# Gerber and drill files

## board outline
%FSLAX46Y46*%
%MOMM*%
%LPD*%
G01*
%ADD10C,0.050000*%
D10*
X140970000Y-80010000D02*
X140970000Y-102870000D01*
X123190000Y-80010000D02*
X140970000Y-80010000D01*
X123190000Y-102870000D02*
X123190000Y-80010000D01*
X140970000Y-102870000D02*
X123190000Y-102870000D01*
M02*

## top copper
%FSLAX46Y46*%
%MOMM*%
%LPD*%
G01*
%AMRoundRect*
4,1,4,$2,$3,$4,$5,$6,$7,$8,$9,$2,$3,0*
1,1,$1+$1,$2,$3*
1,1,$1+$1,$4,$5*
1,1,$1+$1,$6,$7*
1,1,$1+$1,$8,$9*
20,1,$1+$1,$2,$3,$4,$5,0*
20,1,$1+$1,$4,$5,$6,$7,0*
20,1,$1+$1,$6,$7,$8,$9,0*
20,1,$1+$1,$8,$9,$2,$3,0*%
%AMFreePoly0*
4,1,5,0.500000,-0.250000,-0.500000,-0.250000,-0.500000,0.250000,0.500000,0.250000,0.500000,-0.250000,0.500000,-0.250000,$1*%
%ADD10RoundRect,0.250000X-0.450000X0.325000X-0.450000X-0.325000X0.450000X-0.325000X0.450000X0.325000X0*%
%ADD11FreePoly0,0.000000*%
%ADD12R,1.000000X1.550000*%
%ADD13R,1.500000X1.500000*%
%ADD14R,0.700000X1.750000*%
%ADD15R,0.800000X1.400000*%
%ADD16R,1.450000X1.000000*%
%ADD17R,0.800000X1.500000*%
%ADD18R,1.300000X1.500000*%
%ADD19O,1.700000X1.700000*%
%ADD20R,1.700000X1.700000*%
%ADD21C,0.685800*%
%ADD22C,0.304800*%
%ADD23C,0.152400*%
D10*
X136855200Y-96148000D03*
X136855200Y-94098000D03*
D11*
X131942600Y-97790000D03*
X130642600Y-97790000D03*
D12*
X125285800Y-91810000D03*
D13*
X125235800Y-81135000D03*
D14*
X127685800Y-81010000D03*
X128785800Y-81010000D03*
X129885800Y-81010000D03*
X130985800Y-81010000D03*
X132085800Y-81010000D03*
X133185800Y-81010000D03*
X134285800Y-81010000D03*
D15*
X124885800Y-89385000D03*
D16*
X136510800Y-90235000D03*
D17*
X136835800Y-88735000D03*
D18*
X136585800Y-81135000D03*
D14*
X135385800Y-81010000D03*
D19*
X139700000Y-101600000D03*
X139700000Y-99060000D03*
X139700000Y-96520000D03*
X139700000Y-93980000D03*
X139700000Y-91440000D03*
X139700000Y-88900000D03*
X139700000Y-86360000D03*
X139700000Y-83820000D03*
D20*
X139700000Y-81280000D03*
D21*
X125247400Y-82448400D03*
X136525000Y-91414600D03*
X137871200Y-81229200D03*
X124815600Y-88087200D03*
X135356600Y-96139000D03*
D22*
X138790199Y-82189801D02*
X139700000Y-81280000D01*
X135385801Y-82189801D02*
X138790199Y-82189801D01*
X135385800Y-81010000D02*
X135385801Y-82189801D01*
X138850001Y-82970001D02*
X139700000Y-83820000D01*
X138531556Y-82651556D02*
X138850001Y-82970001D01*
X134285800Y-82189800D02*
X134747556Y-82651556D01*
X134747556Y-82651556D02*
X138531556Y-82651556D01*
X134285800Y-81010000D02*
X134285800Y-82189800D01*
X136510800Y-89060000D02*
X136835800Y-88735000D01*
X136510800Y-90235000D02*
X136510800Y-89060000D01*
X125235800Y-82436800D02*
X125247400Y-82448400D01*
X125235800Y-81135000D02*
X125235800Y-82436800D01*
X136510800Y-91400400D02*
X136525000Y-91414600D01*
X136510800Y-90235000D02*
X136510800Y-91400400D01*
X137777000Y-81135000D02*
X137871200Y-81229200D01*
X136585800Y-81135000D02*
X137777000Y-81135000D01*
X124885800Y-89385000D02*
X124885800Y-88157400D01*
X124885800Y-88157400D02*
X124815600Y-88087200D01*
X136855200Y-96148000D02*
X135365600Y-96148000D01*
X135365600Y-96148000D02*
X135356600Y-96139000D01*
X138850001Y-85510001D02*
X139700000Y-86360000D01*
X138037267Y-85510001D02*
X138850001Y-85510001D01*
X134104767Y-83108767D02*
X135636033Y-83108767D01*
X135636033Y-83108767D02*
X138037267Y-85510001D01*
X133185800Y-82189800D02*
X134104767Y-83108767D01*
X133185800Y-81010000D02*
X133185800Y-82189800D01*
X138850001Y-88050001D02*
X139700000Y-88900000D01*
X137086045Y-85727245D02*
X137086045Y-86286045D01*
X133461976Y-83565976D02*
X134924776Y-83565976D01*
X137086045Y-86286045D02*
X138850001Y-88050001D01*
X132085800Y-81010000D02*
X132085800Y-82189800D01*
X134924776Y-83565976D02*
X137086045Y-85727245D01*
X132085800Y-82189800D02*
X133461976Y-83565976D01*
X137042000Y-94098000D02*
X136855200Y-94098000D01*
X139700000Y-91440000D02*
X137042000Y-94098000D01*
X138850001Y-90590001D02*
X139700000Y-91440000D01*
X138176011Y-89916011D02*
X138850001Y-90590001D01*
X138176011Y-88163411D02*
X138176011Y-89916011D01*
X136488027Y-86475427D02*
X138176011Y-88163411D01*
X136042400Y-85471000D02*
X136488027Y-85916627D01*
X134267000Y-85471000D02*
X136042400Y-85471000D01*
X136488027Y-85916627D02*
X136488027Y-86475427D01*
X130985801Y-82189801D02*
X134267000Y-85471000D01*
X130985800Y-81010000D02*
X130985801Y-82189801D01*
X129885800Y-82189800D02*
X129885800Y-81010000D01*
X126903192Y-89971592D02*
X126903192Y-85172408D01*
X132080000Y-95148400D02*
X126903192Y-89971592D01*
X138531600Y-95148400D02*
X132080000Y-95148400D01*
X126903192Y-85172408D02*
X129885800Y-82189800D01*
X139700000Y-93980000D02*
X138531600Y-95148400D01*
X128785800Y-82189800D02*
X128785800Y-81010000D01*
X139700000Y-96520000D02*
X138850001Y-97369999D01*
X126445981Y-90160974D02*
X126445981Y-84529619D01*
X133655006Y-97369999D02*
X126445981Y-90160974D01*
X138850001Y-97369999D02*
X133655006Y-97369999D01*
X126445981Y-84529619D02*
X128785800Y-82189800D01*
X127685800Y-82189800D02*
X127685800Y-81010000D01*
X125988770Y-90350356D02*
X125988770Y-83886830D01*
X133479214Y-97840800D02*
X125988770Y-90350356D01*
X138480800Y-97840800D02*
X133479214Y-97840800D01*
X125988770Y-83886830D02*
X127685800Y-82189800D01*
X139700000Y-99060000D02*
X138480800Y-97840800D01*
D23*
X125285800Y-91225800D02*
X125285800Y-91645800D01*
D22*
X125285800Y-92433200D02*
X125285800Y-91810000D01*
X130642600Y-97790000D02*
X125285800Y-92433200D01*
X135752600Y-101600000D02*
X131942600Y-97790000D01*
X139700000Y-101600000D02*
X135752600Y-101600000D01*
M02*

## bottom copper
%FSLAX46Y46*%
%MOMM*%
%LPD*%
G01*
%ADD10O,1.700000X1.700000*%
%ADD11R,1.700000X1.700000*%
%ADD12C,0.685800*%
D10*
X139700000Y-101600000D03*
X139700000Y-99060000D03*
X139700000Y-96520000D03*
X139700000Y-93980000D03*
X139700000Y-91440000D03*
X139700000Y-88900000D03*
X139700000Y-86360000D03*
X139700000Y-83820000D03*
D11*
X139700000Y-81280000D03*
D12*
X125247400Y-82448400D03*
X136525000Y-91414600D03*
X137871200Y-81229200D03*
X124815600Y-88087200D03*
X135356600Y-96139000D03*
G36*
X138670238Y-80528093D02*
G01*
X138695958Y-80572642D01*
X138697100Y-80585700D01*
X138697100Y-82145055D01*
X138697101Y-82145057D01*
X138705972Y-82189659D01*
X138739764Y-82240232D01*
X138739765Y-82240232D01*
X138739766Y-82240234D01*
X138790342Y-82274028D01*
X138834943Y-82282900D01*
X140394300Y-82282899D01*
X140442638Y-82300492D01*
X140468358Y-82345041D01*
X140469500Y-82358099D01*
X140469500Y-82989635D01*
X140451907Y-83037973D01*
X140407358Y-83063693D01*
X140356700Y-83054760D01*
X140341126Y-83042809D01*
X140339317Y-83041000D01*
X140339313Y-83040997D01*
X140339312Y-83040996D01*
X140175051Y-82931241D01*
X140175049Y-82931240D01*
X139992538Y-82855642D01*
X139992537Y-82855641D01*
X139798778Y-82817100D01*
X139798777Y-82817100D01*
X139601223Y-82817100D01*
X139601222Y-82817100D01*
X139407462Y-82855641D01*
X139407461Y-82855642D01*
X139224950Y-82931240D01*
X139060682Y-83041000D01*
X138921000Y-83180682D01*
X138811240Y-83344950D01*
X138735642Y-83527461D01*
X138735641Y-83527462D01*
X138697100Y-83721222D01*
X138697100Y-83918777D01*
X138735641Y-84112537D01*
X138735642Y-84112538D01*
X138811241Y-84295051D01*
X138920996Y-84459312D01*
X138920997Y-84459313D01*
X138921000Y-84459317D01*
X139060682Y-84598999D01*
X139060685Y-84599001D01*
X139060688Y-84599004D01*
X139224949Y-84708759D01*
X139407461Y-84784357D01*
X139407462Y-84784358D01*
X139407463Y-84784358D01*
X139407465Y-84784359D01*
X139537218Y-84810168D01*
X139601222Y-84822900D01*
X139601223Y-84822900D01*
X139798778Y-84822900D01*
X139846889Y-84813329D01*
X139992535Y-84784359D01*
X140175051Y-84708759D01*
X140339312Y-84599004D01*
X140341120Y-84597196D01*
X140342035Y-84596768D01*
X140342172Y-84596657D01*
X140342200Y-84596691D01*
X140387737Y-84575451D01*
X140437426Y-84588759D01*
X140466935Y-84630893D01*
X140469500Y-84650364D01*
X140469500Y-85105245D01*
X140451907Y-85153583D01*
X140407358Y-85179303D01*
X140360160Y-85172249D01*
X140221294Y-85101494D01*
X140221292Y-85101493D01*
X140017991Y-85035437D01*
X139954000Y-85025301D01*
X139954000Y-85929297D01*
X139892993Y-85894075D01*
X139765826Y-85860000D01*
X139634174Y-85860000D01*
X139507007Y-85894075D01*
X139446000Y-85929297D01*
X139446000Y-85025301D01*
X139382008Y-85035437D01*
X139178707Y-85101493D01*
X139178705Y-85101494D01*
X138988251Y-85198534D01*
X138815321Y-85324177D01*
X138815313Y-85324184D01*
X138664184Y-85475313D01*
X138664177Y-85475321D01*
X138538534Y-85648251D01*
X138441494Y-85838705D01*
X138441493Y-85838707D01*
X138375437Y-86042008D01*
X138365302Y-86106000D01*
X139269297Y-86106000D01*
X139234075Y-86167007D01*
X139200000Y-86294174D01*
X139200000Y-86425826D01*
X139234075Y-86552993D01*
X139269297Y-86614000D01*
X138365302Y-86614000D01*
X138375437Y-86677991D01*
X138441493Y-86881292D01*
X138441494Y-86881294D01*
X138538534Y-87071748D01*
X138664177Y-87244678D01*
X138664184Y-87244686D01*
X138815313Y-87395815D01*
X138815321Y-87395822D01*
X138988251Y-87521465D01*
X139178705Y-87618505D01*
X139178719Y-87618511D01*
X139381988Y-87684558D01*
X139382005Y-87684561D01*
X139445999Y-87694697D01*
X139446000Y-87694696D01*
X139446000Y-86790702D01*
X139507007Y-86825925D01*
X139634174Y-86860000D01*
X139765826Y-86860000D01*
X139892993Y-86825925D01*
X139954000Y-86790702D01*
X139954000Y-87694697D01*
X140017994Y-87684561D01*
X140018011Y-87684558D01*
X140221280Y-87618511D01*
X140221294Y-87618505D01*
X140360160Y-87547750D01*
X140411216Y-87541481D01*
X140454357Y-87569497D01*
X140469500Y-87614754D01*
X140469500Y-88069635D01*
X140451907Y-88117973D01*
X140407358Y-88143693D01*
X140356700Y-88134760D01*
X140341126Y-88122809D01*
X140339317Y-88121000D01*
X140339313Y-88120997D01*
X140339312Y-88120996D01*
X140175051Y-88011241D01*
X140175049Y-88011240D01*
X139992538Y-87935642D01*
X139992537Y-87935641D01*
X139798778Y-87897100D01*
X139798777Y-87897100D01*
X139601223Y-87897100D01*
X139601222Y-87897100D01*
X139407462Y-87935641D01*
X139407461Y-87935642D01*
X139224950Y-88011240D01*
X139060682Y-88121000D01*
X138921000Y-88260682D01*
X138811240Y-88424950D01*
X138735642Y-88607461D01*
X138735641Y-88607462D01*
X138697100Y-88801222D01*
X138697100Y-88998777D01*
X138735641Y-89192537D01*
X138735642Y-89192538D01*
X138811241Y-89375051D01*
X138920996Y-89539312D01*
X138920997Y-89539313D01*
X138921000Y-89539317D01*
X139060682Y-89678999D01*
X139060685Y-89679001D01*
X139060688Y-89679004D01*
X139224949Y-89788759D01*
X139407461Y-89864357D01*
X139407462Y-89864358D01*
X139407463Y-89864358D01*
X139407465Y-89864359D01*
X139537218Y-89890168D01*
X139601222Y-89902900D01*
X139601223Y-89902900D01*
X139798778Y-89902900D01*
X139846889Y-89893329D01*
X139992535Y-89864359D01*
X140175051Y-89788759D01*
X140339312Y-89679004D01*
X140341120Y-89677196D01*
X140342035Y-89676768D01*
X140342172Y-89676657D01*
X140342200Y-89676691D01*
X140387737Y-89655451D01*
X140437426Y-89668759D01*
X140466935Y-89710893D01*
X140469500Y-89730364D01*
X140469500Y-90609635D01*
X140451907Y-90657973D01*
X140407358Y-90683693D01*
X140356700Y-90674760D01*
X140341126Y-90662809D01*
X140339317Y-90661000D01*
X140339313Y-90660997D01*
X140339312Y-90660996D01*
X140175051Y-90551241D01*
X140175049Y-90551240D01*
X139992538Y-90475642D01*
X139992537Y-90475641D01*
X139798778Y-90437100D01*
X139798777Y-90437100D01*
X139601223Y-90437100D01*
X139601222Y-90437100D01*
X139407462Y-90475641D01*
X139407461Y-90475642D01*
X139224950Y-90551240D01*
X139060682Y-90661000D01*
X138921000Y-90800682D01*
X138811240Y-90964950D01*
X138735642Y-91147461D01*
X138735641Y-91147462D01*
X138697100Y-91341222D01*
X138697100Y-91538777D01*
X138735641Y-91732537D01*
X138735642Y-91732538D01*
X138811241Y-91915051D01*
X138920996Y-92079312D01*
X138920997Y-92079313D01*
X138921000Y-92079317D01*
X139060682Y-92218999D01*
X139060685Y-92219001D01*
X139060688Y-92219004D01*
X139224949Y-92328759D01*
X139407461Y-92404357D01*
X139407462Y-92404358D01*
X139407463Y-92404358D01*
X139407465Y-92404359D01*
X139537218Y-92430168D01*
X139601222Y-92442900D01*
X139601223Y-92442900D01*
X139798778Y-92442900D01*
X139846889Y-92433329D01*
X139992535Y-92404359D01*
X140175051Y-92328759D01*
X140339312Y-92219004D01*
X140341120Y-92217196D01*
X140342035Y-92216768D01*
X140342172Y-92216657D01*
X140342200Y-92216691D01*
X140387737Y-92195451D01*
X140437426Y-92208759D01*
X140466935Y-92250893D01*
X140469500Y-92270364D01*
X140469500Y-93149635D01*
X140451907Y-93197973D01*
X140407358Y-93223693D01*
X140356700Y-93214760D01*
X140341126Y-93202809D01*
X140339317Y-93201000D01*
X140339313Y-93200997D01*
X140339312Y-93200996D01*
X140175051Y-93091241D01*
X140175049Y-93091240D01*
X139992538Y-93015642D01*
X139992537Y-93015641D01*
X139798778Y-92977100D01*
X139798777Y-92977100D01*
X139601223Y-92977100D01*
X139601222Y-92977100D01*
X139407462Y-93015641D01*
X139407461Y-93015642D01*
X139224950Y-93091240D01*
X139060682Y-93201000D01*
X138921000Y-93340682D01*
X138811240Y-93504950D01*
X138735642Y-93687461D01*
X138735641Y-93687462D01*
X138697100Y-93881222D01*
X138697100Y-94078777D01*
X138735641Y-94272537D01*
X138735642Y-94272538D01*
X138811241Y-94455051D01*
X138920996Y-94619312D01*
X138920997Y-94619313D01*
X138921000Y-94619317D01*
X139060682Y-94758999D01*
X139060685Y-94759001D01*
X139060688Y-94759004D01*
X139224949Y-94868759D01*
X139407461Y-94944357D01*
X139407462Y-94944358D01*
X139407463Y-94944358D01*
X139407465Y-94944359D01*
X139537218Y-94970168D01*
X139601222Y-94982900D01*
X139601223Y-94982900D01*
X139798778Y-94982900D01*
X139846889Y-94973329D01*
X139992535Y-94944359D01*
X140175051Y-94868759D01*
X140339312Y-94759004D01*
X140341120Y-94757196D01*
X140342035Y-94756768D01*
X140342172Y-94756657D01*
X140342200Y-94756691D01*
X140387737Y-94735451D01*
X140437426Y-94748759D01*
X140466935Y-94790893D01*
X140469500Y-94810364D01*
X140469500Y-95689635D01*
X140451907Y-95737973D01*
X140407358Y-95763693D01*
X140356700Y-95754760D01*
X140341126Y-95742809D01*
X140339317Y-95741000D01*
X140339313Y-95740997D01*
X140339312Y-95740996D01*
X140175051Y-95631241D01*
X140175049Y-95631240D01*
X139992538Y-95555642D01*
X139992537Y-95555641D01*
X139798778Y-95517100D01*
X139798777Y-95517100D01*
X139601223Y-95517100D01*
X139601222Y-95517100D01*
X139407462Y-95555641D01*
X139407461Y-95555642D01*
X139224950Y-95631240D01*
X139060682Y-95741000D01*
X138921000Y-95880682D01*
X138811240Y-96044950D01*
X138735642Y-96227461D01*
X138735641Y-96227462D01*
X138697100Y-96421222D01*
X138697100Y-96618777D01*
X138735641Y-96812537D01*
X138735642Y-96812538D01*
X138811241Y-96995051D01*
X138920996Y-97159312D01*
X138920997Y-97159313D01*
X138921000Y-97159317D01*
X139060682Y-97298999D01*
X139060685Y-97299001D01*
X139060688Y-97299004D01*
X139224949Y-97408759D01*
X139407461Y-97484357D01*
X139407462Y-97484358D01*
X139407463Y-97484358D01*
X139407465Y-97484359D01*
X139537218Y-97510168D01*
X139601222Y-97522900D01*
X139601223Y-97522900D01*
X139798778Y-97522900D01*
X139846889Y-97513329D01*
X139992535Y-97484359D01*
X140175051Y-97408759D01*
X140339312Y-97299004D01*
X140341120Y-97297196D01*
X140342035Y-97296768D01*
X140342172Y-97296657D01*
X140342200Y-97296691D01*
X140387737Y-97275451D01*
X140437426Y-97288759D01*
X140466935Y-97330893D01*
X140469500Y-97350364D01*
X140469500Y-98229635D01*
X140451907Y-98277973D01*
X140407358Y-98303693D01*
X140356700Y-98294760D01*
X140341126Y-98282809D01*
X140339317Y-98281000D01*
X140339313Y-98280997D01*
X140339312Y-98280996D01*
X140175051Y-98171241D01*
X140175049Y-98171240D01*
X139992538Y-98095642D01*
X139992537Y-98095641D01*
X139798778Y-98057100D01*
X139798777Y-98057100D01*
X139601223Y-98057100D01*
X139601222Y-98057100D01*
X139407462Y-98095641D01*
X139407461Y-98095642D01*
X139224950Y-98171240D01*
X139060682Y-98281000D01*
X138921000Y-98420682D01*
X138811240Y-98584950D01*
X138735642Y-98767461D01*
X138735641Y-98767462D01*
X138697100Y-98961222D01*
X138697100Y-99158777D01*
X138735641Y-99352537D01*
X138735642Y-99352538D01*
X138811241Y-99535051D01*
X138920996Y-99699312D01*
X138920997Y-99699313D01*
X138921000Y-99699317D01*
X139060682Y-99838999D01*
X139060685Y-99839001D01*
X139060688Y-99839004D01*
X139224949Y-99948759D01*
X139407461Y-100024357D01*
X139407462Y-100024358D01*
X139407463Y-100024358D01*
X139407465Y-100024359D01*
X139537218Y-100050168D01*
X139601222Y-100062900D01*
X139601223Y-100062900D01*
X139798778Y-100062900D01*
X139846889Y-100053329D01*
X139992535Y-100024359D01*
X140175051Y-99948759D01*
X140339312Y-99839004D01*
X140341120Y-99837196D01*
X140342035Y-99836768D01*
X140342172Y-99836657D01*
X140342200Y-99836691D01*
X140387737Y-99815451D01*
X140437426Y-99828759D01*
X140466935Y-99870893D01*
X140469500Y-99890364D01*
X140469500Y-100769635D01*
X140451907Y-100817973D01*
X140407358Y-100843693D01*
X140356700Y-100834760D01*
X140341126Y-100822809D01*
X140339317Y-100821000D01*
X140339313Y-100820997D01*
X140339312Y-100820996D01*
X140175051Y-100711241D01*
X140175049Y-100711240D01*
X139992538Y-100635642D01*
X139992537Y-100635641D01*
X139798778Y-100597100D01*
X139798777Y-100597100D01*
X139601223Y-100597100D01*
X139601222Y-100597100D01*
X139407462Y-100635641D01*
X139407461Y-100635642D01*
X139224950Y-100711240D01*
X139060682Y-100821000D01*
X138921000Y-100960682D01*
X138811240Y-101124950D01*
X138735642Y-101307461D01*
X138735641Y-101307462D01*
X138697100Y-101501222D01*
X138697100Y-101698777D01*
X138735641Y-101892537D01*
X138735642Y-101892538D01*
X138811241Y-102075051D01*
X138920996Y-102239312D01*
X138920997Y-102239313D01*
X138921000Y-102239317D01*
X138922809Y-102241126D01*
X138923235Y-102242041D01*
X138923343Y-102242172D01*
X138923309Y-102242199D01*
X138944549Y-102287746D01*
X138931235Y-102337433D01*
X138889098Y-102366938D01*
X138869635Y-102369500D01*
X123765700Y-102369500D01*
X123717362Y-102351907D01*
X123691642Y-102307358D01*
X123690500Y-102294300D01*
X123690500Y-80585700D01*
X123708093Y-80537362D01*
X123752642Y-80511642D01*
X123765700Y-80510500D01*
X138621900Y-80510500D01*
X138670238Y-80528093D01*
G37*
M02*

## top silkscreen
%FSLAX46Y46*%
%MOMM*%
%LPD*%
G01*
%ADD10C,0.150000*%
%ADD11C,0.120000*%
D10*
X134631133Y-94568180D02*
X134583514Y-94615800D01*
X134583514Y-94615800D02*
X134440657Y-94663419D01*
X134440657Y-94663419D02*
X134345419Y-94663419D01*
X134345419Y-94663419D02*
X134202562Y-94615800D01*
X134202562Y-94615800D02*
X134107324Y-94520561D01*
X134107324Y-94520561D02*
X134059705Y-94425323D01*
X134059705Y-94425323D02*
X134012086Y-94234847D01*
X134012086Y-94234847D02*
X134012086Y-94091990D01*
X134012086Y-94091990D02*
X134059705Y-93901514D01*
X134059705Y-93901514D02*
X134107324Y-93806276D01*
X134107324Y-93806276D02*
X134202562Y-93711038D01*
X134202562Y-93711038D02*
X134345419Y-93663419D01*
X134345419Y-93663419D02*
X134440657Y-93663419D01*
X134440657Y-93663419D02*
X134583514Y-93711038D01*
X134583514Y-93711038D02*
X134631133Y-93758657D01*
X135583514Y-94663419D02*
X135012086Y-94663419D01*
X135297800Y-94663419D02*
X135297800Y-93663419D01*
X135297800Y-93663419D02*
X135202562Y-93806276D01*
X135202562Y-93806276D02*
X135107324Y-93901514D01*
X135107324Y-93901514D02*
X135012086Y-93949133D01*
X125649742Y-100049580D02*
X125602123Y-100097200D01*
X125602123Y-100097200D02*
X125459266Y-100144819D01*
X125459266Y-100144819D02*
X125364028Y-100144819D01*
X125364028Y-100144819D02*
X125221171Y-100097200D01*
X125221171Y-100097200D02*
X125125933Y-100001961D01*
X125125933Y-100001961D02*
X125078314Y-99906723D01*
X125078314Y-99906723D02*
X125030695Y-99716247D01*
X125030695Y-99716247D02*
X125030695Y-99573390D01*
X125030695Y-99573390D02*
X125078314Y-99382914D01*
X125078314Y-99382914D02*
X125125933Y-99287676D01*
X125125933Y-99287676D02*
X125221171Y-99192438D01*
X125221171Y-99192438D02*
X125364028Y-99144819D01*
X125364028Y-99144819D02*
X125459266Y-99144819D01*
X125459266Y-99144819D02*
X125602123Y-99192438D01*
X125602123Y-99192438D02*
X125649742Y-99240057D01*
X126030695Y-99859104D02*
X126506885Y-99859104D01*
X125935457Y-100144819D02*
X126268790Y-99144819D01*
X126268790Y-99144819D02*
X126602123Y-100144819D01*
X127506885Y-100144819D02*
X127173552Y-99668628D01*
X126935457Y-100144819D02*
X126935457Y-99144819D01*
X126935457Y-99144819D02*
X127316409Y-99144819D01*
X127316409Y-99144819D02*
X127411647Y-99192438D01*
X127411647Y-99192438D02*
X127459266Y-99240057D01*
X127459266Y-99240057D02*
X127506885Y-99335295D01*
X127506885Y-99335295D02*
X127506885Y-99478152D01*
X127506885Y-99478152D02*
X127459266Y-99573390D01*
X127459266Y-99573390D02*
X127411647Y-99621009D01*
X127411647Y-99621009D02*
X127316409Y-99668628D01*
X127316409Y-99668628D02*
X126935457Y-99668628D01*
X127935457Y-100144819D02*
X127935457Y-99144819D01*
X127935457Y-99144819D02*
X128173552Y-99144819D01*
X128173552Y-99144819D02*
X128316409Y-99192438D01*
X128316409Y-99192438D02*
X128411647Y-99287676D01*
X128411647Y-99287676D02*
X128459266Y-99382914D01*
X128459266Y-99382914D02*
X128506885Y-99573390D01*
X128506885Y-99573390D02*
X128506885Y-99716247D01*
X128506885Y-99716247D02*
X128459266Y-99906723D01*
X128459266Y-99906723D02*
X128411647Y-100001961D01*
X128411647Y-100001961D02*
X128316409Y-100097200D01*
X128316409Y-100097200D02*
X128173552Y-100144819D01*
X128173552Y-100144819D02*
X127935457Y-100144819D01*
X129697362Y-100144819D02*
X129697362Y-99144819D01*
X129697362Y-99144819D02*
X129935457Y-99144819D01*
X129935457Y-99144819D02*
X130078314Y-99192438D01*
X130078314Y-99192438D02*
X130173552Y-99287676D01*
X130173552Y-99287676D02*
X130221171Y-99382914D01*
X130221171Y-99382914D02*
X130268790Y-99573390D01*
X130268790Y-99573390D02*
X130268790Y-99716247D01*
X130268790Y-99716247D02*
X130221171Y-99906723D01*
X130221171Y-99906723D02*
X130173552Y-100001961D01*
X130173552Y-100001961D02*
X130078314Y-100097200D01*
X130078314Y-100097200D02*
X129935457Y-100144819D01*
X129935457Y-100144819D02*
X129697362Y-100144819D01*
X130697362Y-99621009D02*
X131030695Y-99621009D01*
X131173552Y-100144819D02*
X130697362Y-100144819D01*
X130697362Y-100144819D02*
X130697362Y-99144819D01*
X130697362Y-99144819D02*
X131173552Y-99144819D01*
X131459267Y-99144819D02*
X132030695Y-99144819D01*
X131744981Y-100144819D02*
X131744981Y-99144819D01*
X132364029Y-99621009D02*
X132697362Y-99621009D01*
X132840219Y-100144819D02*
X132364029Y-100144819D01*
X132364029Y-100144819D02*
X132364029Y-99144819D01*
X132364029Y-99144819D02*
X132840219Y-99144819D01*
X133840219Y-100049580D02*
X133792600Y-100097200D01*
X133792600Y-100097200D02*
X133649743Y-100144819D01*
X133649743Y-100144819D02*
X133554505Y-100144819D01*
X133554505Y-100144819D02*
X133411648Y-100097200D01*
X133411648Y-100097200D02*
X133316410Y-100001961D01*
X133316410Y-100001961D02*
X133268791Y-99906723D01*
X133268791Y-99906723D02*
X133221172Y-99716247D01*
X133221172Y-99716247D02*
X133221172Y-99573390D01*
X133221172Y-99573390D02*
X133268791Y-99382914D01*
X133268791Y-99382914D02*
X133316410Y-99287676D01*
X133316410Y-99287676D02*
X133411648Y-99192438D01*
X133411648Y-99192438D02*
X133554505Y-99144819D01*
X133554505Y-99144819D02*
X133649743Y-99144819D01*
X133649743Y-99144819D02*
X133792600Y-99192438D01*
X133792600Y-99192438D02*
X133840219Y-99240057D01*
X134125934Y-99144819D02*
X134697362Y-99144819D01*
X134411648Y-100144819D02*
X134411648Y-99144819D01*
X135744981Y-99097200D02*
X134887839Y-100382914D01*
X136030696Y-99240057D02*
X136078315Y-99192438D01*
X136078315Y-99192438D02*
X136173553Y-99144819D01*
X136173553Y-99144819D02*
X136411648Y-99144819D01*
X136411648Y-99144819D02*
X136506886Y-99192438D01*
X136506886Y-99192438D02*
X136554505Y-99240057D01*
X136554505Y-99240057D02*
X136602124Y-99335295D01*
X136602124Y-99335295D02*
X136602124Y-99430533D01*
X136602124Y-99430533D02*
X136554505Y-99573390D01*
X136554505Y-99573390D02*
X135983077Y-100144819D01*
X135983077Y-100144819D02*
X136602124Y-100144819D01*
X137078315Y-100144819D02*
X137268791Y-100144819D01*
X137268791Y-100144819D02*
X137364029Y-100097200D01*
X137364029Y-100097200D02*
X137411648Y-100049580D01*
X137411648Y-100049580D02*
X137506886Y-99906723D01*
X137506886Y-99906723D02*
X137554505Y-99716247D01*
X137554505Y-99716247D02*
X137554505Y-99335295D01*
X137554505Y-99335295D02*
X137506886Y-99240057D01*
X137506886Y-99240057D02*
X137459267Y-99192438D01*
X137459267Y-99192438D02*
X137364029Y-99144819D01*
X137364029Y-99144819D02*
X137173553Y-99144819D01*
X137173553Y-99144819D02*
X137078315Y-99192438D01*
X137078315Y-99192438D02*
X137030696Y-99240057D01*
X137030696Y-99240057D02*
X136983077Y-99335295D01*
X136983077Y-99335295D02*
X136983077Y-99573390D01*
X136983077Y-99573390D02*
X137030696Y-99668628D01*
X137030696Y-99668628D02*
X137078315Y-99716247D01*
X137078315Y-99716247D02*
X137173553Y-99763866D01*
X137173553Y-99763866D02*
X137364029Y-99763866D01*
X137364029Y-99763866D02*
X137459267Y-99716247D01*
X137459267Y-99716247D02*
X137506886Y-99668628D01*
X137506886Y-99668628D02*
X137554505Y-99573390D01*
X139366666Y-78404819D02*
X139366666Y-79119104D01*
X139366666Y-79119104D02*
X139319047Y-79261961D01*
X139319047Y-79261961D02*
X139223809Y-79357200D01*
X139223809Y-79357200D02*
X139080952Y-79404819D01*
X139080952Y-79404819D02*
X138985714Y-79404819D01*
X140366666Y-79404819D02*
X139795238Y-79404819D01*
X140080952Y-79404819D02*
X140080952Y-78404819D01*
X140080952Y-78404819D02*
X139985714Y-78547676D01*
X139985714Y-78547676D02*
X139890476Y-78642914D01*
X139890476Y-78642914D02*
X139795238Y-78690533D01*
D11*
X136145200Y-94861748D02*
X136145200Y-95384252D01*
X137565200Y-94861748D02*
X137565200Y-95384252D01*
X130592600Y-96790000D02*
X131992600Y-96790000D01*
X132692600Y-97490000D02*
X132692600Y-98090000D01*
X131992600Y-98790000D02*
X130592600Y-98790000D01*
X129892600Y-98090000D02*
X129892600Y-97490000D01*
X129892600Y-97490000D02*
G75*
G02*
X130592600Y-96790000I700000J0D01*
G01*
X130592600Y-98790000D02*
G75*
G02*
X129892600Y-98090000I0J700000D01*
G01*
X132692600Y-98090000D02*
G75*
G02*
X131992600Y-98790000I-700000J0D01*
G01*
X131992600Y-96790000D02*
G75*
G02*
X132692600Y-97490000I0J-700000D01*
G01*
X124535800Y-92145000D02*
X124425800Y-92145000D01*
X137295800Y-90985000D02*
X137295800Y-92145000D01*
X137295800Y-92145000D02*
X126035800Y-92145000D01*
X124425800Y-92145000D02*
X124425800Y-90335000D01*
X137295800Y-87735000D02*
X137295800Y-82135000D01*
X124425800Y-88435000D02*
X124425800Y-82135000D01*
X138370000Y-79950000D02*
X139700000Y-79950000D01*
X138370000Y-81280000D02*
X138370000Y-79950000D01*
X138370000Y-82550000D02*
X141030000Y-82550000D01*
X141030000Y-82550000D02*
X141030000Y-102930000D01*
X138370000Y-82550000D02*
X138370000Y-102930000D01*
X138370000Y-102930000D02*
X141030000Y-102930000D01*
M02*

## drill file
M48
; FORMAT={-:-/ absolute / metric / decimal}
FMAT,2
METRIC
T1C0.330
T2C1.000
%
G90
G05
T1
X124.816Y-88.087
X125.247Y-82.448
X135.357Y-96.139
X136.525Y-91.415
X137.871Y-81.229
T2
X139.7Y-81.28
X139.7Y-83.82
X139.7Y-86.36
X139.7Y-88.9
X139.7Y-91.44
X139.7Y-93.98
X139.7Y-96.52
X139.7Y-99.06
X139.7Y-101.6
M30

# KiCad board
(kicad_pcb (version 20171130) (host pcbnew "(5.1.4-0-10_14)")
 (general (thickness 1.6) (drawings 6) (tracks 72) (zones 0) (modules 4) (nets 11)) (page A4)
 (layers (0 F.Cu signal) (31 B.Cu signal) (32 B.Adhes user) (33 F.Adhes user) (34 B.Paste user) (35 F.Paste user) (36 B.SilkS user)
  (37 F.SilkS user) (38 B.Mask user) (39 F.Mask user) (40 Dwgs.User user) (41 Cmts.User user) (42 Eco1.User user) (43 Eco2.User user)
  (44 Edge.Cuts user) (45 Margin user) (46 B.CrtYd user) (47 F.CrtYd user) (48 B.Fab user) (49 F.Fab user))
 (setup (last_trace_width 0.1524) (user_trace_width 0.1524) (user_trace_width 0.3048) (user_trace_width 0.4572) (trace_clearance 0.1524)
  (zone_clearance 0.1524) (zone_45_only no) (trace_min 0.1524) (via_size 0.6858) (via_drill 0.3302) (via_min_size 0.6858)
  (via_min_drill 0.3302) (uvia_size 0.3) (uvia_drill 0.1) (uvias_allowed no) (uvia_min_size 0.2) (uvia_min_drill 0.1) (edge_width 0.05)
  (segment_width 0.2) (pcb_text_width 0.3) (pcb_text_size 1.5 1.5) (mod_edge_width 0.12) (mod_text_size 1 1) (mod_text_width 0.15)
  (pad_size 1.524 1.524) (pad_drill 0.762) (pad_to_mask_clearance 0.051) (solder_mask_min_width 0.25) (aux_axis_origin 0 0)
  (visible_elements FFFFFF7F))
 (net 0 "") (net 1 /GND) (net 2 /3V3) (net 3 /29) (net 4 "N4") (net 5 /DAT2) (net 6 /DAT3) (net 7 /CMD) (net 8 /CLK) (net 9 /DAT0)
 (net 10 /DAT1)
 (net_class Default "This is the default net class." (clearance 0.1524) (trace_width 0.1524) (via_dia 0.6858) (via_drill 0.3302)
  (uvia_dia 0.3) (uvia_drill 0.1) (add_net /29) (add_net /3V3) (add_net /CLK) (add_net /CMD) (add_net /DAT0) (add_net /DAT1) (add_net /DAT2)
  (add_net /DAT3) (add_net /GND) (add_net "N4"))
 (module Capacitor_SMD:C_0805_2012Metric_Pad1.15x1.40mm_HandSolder (layer F.Cu) (at 136.8552 95.123 270)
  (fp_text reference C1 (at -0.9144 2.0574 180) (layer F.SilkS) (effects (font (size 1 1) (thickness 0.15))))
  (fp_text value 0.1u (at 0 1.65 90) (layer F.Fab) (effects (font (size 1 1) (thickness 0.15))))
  (fp_line (start -0.261252 0.71) (end 0.261252 0.71) (layer F.SilkS) (width 0.12))
  (fp_line (start -0.261252 -0.71) (end 0.261252 -0.71) (layer F.SilkS) (width 0.12))
  (pad 2 smd roundrect (at 1.025 0 270) (size 1.15 1.4) (layers F.Cu F.Paste F.Mask) (roundrect_rratio 0.217391) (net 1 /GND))
  (pad 1 smd roundrect (at -1.025 0 270) (size 1.15 1.4) (layers F.Cu F.Paste F.Mask) (roundrect_rratio 0.217391) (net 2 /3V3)))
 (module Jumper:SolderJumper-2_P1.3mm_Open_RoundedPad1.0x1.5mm (layer F.Cu) (at 131.2926 97.79)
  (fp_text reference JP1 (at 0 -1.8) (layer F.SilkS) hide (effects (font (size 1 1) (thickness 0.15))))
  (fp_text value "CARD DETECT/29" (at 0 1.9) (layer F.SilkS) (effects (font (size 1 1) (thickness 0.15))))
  (fp_line (start -0.7 -1) (end 0.7 -1) (layer F.SilkS) (width 0.12))
  (fp_line (start 1.4 -0.3) (end 1.4 0.3) (layer F.SilkS) (width 0.12))
  (fp_line (start 0.7 1) (end -0.7 1) (layer F.SilkS) (width 0.12))
  (fp_line (start -1.4 0.3) (end -1.4 -0.3) (layer F.SilkS) (width 0.12))
  (fp_arc (start -0.7 -0.3) (end -0.7 -1) (angle -90) (layer F.SilkS) (width 0.12))
  (fp_arc (start -0.7 0.3) (end -1.4 0.3) (angle -90) (layer F.SilkS) (width 0.12))
  (fp_arc (start 0.7 0.3) (end 0.7 1) (angle -90) (layer F.SilkS) (width 0.12))
  (fp_arc (start 0.7 -0.3) (end 1.4 -0.3) (angle -90) (layer F.SilkS) (width 0.12))
  (pad 2 smd custom (at 0.65 0) (size 1 0.5) (layers F.Cu F.Mask) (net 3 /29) (zone_connect 2) (options (clearance outline) (anchor rect))
   (primitives))
  (pad 1 smd custom (at -0.65 0) (size 1 0.5) (layers F.Cu F.Mask) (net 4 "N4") (zone_connect 2) (options (clearance outline) (anchor rect))
   (primitives)))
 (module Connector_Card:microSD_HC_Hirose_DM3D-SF (layer F.Cu) (at 130.8608 86.36 180)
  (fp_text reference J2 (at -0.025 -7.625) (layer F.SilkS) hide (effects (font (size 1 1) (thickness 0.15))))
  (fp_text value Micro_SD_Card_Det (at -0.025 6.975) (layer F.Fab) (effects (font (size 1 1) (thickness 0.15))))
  (fp_line (start 6.325 -5.785) (end 6.435 -5.785) (layer F.SilkS) (width 0.12))
  (fp_line (start -6.435 -4.625) (end -6.435 -5.785) (layer F.SilkS) (width 0.12))
  (fp_line (start -6.435 -5.785) (end 4.825 -5.785) (layer F.SilkS) (width 0.12))
  (fp_line (start 6.435 -5.785) (end 6.435 -3.975) (layer F.SilkS) (width 0.12))
  (fp_line (start -6.435 -1.375) (end -6.435 4.225) (layer F.SilkS) (width 0.12))
  (fp_line (start 6.435 -2.075) (end 6.435 4.225) (layer F.SilkS) (width 0.12))
  (pad 10 smd rect (at 5.575 -5.45 180) (size 1 1.55) (layers F.Cu F.Paste F.Mask) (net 4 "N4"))
  (pad 11 smd rect (at 5.625 5.225 180) (size 1.5 1.5) (layers F.Cu F.Paste F.Mask) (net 1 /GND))
  (pad 1 smd rect (at 3.175 5.35 180) (size 0.7 1.75) (layers F.Cu F.Paste F.Mask) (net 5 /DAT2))
  (pad 2 smd rect (at 2.075 5.35 180) (size 0.7 1.75) (layers F.Cu F.Paste F.Mask) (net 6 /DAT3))
  (pad 3 smd rect (at 0.975 5.35 180) (size 0.7 1.75) (layers F.Cu F.Paste F.Mask) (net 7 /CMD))
  (pad 4 smd rect (at -0.125 5.35 180) (size 0.7 1.75) (layers F.Cu F.Paste F.Mask) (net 2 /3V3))
  (pad 5 smd rect (at -1.225 5.35 180) (size 0.7 1.75) (layers F.Cu F.Paste F.Mask) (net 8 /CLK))
  (pad 6 smd rect (at -2.325 5.35 180) (size 0.7 1.75) (layers F.Cu F.Paste F.Mask) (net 1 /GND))
  (pad 7 smd rect (at -3.425 5.35 180) (size 0.7 1.75) (layers F.Cu F.Paste F.Mask) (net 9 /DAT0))
  (pad 11 smd rect (at 5.975 -3.025 180) (size 0.8 1.4) (layers F.Cu F.Paste F.Mask) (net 1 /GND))
  (pad 9 smd rect (at -5.65 -3.875 180) (size 1.45 1) (layers F.Cu F.Paste F.Mask) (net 1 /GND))
  (pad 11 smd rect (at -5.975 -2.375 180) (size 0.8 1.5) (layers F.Cu F.Paste F.Mask) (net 1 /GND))
  (pad 11 smd rect (at -5.725 5.225 180) (size 1.3 1.5) (layers F.Cu F.Paste F.Mask) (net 1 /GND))
  (pad 8 smd rect (at -4.525 5.35 180) (size 0.7 1.75) (layers F.Cu F.Paste F.Mask) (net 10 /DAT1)))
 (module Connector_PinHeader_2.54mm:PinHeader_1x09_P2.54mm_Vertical (layer F.Cu) (at 139.7 81.28)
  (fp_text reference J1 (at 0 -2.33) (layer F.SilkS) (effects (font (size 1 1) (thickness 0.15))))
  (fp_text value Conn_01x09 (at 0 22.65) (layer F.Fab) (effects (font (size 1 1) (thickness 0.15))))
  (fp_line (start -1.33 -1.33) (end 0 -1.33) (layer F.SilkS) (width 0.12))
  (fp_line (start -1.33 0) (end -1.33 -1.33) (layer F.SilkS) (width 0.12))
  (fp_line (start -1.33 1.27) (end 1.33 1.27) (layer F.SilkS) (width 0.12))
  (fp_line (start 1.33 1.27) (end 1.33 21.65) (layer F.SilkS) (width 0.12))
  (fp_line (start -1.33 1.27) (end -1.33 21.65) (layer F.SilkS) (width 0.12))
  (fp_line (start -1.33 21.65) (end 1.33 21.65) (layer F.SilkS) (width 0.12))
  (pad 9 thru_hole oval (at 0 20.32) (size 1.7 1.7) (drill 1) (layers *.Cu *.Mask) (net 3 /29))
  (pad 8 thru_hole oval (at 0 17.78) (size 1.7 1.7) (drill 1) (layers *.Cu *.Mask) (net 5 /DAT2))
  (pad 7 thru_hole oval (at 0 15.24) (size 1.7 1.7) (drill 1) (layers *.Cu *.Mask) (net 6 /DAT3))
  (pad 6 thru_hole oval (at 0 12.7) (size 1.7 1.7) (drill 1) (layers *.Cu *.Mask) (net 7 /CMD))
  (pad 5 thru_hole oval (at 0 10.16) (size 1.7 1.7) (drill 1) (layers *.Cu *.Mask) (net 2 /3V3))
  (pad 4 thru_hole oval (at 0 7.62) (size 1.7 1.7) (drill 1) (layers *.Cu *.Mask) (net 8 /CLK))
  (pad 3 thru_hole oval (at 0 5.08) (size 1.7 1.7) (drill 1) (layers *.Cu *.Mask) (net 1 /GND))
  (pad 2 thru_hole oval (at 0 2.54) (size 1.7 1.7) (drill 1) (layers *.Cu *.Mask) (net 9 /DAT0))
  (pad 1 thru_hole rect (at 0 0) (size 1.7 1.7) (drill 1) (layers *.Cu *.Mask) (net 10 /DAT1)))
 (gr_line (start 140.97 80.01) (end 140.97 102.87) (layer Edge.Cuts) (width 0.05))
 (gr_line (start 123.19 80.01) (end 140.97 80.01) (layer Edge.Cuts) (width 0.05))
 (gr_line (start 123.19 102.87) (end 123.19 80.01) (layer Edge.Cuts) (width 0.05))
 (gr_line (start 140.97 102.87) (end 123.19 102.87) (layer Edge.Cuts) (width 0.05))
 (segment (start 138.790199 82.189801) (end 139.7 81.28) (width 0.3048) (layer F.Cu) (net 10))
 (segment (start 135.385801 82.189801) (end 138.790199 82.189801) (width 0.3048) (layer F.Cu) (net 10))
 (segment (start 135.3858 81.01) (end 135.385801 82.189801) (width 0.3048) (layer F.Cu) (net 10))
 (segment (start 138.850001 82.970001) (end 139.7 83.82) (width 0.3048) (layer F.Cu) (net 9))
 (segment (start 138.531556 82.651556) (end 138.850001 82.970001) (width 0.3048) (layer F.Cu) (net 9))
 (segment (start 134.2858 82.1898) (end 134.747556 82.651556) (width 0.3048) (layer F.Cu) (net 9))
 (segment (start 134.747556 82.651556) (end 138.531556 82.651556) (width 0.3048) (layer F.Cu) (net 9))
 (segment (start 134.2858 81.01) (end 134.2858 82.1898) (width 0.3048) (layer F.Cu) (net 9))
 (segment (start 136.5108 89.06) (end 136.8358 88.735) (width 0.3048) (layer F.Cu) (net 1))
 (segment (start 136.5108 90.235) (end 136.5108 89.06) (width 0.3048) (layer F.Cu) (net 1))
 (segment (start 125.2358 82.4368) (end 125.2474 82.4484) (width 0.3048) (layer F.Cu) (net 1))
 (via (at 125.2474 82.4484) (size 0.6858) (drill 0.3302) (layers F.Cu B.Cu) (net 1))
 (segment (start 125.2358 81.135) (end 125.2358 82.4368) (width 0.3048) (layer F.Cu) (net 1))
 (via (at 136.525 91.4146) (size 0.6858) (drill 0.3302) (layers F.Cu B.Cu) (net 1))
 (segment (start 136.5108 91.4004) (end 136.525 91.4146) (width 0.3048) (layer F.Cu) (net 1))
 (segment (start 136.5108 90.235) (end 136.5108 91.4004) (width 0.3048) (layer F.Cu) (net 1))
 (via (at 137.8712 81.2292) (size 0.6858) (drill 0.3302) (layers F.Cu B.Cu) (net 1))
 (segment (start 137.777 81.135) (end 137.8712 81.2292) (width 0.3048) (layer F.Cu) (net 1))
 (segment (start 136.5858 81.135) (end 137.777 81.135) (width 0.3048) (layer F.Cu) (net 1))
 (via (at 124.8156 88.0872) (size 0.6858) (drill 0.3302) (layers F.Cu B.Cu) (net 1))
 (segment (start 124.8858 89.385) (end 124.8858 88.1574) (width 0.3048) (layer F.Cu) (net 1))
 (segment (start 124.8858 88.1574) (end 124.8156 88.0872) (width 0.3048) (layer F.Cu) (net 1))
 (via (at 135.3566 96.139) (size 0.6858) (drill 0.3302) (layers F.Cu B.Cu) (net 1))
 (segment (start 136.8552 96.148) (end 135.3656 96.148) (width 0.3048) (layer F.Cu) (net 1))
 (segment (start 135.3656 96.148) (end 135.3566 96.139) (width 0.3048) (layer F.Cu) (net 1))
 (segment (start 138.850001 85.510001) (end 139.7 86.36) (width 0.3048) (layer F.Cu) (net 1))
 (segment (start 138.037267 85.510001) (end 138.850001 85.510001) (width 0.3048) (layer F.Cu) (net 1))
 (segment (start 134.104767 83.108767) (end 135.636033 83.108767) (width 0.3048) (layer F.Cu) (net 1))
 (segment (start 135.636033 83.108767) (end 138.037267 85.510001) (width 0.3048) (layer F.Cu) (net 1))
 (segment (start 133.1858 82.1898) (end 134.104767 83.108767) (width 0.3048) (layer F.Cu) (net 1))
 (segment (start 133.1858 81.01) (end 133.1858 82.1898) (width 0.3048) (layer F.Cu) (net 1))
 (segment (start 138.850001 88.050001) (end 139.7 88.9) (width 0.3048) (layer F.Cu) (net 8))
 (segment (start 137.086045 85.727245) (end 137.086045 86.286045) (width 0.3048) (layer F.Cu) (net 8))
 (segment (start 133.461976 83.565976) (end 134.924776 83.565976) (width 0.3048) (layer F.Cu) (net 8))
 (segment (start 137.086045 86.286045) (end 138.850001 88.050001) (width 0.3048) (layer F.Cu) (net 8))
 (segment (start 132.0858 81.01) (end 132.0858 82.1898) (width 0.3048) (layer F.Cu) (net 8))
 (segment (start 134.924776 83.565976) (end 137.086045 85.727245) (width 0.3048) (layer F.Cu) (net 8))
 (segment (start 132.0858 82.1898) (end 133.461976 83.565976) (width 0.3048) (layer F.Cu) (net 8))
 (segment (start 137.042 94.098) (end 136.8552 94.098) (width 0.3048) (layer F.Cu) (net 2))
 (segment (start 139.7 91.44) (end 137.042 94.098) (width 0.3048) (layer F.Cu) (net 2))
 (segment (start 138.850001 90.590001) (end 139.7 91.44) (width 0.3048) (layer F.Cu) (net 2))
 (segment (start 138.176011 89.916011) (end 138.850001 90.590001) (width 0.3048) (layer F.Cu) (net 2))
 (segment (start 138.176011 88.163411) (end 138.176011 89.916011) (width 0.3048) (layer F.Cu) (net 2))
 (segment (start 136.488027 86.475427) (end 138.176011 88.163411) (width 0.3048) (layer F.Cu) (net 2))
 (segment (start 136.0424 85.471) (end 136.488027 85.916627) (width 0.3048) (layer F.Cu) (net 2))
 (segment (start 134.267 85.471) (end 136.0424 85.471) (width 0.3048) (layer F.Cu) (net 2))
 (segment (start 136.488027 85.916627) (end 136.488027 86.475427) (width 0.3048) (layer F.Cu) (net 2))
 (segment (start 130.985801 82.189801) (end 134.267 85.471) (width 0.3048) (layer F.Cu) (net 2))
 (segment (start 130.9858 81.01) (end 130.985801 82.189801) (width 0.3048) (layer F.Cu) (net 2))
 (segment (start 129.8858 82.1898) (end 129.8858 81.01) (width 0.3048) (layer F.Cu) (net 7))
 (segment (start 126.903192 89.971592) (end 126.903192 85.172408) (width 0.3048) (layer F.Cu) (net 7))
 (segment (start 132.08 95.1484) (end 126.903192 89.971592) (width 0.3048) (layer F.Cu) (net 7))
 (segment (start 138.5316 95.1484) (end 132.08 95.1484) (width 0.3048) (layer F.Cu) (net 7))
 (segment (start 126.903192 85.172408) (end 129.8858 82.1898) (width 0.3048) (layer F.Cu) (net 7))
 (segment (start 139.7 93.98) (end 138.5316 95.1484) (width 0.3048) (layer F.Cu) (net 7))
 (segment (start 128.7858 82.1898) (end 128.7858 81.01) (width 0.3048) (layer F.Cu) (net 6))
 (segment (start 139.7 96.52) (end 138.850001 97.369999) (width 0.3048) (layer F.Cu) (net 6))
 (segment (start 126.445981 90.160974) (end 126.445981 84.529619) (width 0.3048) (layer F.Cu) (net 6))
 (segment (start 133.655006 97.369999) (end 126.445981 90.160974) (width 0.3048) (layer F.Cu) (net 6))
 (segment (start 138.850001 97.369999) (end 133.655006 97.369999) (width 0.3048) (layer F.Cu) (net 6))
 (segment (start 126.445981 84.529619) (end 128.7858 82.1898) (width 0.3048) (layer F.Cu) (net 6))
 (segment (start 127.6858 82.1898) (end 127.6858 81.01) (width 0.3048) (layer F.Cu) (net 5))
 (segment (start 125.98877 90.350356) (end 125.98877 83.88683) (width 0.3048) (layer F.Cu) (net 5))
 (segment (start 133.479214 97.8408) (end 125.98877 90.350356) (width 0.3048) (layer F.Cu) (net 5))
 (segment (start 138.4808 97.8408) (end 133.479214 97.8408) (width 0.3048) (layer F.Cu) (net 5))
 (segment (start 125.98877 83.88683) (end 127.6858 82.1898) (width 0.3048) (layer F.Cu) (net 5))
 (segment (start 139.7 99.06) (end 138.4808 97.8408) (width 0.3048) (layer F.Cu) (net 5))
 (segment (start 125.2858 91.2258) (end 125.2858 91.6458) (width 0.1524) (layer F.Cu) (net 4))
 (segment (start 125.2858 92.4332) (end 125.2858 91.81) (width 0.3048) (layer F.Cu) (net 4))
 (segment (start 130.6426 97.79) (end 125.2858 92.4332) (width 0.3048) (layer F.Cu) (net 4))
 (segment (start 135.7526 101.6) (end 131.9426 97.79) (width 0.3048) (layer F.Cu) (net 3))
 (segment (start 139.7 101.6) (end 135.7526 101.6) (width 0.3048) (layer F.Cu) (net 3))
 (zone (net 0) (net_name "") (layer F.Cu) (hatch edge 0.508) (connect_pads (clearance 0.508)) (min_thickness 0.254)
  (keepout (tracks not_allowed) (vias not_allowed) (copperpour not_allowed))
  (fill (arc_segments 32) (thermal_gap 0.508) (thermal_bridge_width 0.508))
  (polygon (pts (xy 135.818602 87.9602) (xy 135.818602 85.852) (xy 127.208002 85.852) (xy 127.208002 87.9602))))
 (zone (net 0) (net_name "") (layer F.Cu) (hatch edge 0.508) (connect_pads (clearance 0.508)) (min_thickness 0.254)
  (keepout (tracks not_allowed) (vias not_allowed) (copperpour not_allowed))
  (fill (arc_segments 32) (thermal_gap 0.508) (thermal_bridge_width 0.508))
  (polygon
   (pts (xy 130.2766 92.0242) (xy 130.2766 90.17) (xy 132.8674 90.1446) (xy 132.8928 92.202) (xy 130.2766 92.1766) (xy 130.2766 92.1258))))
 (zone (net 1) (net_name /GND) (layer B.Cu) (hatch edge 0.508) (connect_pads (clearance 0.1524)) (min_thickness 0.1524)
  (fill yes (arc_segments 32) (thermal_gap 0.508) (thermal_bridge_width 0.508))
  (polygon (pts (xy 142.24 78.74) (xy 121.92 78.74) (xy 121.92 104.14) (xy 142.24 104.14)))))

